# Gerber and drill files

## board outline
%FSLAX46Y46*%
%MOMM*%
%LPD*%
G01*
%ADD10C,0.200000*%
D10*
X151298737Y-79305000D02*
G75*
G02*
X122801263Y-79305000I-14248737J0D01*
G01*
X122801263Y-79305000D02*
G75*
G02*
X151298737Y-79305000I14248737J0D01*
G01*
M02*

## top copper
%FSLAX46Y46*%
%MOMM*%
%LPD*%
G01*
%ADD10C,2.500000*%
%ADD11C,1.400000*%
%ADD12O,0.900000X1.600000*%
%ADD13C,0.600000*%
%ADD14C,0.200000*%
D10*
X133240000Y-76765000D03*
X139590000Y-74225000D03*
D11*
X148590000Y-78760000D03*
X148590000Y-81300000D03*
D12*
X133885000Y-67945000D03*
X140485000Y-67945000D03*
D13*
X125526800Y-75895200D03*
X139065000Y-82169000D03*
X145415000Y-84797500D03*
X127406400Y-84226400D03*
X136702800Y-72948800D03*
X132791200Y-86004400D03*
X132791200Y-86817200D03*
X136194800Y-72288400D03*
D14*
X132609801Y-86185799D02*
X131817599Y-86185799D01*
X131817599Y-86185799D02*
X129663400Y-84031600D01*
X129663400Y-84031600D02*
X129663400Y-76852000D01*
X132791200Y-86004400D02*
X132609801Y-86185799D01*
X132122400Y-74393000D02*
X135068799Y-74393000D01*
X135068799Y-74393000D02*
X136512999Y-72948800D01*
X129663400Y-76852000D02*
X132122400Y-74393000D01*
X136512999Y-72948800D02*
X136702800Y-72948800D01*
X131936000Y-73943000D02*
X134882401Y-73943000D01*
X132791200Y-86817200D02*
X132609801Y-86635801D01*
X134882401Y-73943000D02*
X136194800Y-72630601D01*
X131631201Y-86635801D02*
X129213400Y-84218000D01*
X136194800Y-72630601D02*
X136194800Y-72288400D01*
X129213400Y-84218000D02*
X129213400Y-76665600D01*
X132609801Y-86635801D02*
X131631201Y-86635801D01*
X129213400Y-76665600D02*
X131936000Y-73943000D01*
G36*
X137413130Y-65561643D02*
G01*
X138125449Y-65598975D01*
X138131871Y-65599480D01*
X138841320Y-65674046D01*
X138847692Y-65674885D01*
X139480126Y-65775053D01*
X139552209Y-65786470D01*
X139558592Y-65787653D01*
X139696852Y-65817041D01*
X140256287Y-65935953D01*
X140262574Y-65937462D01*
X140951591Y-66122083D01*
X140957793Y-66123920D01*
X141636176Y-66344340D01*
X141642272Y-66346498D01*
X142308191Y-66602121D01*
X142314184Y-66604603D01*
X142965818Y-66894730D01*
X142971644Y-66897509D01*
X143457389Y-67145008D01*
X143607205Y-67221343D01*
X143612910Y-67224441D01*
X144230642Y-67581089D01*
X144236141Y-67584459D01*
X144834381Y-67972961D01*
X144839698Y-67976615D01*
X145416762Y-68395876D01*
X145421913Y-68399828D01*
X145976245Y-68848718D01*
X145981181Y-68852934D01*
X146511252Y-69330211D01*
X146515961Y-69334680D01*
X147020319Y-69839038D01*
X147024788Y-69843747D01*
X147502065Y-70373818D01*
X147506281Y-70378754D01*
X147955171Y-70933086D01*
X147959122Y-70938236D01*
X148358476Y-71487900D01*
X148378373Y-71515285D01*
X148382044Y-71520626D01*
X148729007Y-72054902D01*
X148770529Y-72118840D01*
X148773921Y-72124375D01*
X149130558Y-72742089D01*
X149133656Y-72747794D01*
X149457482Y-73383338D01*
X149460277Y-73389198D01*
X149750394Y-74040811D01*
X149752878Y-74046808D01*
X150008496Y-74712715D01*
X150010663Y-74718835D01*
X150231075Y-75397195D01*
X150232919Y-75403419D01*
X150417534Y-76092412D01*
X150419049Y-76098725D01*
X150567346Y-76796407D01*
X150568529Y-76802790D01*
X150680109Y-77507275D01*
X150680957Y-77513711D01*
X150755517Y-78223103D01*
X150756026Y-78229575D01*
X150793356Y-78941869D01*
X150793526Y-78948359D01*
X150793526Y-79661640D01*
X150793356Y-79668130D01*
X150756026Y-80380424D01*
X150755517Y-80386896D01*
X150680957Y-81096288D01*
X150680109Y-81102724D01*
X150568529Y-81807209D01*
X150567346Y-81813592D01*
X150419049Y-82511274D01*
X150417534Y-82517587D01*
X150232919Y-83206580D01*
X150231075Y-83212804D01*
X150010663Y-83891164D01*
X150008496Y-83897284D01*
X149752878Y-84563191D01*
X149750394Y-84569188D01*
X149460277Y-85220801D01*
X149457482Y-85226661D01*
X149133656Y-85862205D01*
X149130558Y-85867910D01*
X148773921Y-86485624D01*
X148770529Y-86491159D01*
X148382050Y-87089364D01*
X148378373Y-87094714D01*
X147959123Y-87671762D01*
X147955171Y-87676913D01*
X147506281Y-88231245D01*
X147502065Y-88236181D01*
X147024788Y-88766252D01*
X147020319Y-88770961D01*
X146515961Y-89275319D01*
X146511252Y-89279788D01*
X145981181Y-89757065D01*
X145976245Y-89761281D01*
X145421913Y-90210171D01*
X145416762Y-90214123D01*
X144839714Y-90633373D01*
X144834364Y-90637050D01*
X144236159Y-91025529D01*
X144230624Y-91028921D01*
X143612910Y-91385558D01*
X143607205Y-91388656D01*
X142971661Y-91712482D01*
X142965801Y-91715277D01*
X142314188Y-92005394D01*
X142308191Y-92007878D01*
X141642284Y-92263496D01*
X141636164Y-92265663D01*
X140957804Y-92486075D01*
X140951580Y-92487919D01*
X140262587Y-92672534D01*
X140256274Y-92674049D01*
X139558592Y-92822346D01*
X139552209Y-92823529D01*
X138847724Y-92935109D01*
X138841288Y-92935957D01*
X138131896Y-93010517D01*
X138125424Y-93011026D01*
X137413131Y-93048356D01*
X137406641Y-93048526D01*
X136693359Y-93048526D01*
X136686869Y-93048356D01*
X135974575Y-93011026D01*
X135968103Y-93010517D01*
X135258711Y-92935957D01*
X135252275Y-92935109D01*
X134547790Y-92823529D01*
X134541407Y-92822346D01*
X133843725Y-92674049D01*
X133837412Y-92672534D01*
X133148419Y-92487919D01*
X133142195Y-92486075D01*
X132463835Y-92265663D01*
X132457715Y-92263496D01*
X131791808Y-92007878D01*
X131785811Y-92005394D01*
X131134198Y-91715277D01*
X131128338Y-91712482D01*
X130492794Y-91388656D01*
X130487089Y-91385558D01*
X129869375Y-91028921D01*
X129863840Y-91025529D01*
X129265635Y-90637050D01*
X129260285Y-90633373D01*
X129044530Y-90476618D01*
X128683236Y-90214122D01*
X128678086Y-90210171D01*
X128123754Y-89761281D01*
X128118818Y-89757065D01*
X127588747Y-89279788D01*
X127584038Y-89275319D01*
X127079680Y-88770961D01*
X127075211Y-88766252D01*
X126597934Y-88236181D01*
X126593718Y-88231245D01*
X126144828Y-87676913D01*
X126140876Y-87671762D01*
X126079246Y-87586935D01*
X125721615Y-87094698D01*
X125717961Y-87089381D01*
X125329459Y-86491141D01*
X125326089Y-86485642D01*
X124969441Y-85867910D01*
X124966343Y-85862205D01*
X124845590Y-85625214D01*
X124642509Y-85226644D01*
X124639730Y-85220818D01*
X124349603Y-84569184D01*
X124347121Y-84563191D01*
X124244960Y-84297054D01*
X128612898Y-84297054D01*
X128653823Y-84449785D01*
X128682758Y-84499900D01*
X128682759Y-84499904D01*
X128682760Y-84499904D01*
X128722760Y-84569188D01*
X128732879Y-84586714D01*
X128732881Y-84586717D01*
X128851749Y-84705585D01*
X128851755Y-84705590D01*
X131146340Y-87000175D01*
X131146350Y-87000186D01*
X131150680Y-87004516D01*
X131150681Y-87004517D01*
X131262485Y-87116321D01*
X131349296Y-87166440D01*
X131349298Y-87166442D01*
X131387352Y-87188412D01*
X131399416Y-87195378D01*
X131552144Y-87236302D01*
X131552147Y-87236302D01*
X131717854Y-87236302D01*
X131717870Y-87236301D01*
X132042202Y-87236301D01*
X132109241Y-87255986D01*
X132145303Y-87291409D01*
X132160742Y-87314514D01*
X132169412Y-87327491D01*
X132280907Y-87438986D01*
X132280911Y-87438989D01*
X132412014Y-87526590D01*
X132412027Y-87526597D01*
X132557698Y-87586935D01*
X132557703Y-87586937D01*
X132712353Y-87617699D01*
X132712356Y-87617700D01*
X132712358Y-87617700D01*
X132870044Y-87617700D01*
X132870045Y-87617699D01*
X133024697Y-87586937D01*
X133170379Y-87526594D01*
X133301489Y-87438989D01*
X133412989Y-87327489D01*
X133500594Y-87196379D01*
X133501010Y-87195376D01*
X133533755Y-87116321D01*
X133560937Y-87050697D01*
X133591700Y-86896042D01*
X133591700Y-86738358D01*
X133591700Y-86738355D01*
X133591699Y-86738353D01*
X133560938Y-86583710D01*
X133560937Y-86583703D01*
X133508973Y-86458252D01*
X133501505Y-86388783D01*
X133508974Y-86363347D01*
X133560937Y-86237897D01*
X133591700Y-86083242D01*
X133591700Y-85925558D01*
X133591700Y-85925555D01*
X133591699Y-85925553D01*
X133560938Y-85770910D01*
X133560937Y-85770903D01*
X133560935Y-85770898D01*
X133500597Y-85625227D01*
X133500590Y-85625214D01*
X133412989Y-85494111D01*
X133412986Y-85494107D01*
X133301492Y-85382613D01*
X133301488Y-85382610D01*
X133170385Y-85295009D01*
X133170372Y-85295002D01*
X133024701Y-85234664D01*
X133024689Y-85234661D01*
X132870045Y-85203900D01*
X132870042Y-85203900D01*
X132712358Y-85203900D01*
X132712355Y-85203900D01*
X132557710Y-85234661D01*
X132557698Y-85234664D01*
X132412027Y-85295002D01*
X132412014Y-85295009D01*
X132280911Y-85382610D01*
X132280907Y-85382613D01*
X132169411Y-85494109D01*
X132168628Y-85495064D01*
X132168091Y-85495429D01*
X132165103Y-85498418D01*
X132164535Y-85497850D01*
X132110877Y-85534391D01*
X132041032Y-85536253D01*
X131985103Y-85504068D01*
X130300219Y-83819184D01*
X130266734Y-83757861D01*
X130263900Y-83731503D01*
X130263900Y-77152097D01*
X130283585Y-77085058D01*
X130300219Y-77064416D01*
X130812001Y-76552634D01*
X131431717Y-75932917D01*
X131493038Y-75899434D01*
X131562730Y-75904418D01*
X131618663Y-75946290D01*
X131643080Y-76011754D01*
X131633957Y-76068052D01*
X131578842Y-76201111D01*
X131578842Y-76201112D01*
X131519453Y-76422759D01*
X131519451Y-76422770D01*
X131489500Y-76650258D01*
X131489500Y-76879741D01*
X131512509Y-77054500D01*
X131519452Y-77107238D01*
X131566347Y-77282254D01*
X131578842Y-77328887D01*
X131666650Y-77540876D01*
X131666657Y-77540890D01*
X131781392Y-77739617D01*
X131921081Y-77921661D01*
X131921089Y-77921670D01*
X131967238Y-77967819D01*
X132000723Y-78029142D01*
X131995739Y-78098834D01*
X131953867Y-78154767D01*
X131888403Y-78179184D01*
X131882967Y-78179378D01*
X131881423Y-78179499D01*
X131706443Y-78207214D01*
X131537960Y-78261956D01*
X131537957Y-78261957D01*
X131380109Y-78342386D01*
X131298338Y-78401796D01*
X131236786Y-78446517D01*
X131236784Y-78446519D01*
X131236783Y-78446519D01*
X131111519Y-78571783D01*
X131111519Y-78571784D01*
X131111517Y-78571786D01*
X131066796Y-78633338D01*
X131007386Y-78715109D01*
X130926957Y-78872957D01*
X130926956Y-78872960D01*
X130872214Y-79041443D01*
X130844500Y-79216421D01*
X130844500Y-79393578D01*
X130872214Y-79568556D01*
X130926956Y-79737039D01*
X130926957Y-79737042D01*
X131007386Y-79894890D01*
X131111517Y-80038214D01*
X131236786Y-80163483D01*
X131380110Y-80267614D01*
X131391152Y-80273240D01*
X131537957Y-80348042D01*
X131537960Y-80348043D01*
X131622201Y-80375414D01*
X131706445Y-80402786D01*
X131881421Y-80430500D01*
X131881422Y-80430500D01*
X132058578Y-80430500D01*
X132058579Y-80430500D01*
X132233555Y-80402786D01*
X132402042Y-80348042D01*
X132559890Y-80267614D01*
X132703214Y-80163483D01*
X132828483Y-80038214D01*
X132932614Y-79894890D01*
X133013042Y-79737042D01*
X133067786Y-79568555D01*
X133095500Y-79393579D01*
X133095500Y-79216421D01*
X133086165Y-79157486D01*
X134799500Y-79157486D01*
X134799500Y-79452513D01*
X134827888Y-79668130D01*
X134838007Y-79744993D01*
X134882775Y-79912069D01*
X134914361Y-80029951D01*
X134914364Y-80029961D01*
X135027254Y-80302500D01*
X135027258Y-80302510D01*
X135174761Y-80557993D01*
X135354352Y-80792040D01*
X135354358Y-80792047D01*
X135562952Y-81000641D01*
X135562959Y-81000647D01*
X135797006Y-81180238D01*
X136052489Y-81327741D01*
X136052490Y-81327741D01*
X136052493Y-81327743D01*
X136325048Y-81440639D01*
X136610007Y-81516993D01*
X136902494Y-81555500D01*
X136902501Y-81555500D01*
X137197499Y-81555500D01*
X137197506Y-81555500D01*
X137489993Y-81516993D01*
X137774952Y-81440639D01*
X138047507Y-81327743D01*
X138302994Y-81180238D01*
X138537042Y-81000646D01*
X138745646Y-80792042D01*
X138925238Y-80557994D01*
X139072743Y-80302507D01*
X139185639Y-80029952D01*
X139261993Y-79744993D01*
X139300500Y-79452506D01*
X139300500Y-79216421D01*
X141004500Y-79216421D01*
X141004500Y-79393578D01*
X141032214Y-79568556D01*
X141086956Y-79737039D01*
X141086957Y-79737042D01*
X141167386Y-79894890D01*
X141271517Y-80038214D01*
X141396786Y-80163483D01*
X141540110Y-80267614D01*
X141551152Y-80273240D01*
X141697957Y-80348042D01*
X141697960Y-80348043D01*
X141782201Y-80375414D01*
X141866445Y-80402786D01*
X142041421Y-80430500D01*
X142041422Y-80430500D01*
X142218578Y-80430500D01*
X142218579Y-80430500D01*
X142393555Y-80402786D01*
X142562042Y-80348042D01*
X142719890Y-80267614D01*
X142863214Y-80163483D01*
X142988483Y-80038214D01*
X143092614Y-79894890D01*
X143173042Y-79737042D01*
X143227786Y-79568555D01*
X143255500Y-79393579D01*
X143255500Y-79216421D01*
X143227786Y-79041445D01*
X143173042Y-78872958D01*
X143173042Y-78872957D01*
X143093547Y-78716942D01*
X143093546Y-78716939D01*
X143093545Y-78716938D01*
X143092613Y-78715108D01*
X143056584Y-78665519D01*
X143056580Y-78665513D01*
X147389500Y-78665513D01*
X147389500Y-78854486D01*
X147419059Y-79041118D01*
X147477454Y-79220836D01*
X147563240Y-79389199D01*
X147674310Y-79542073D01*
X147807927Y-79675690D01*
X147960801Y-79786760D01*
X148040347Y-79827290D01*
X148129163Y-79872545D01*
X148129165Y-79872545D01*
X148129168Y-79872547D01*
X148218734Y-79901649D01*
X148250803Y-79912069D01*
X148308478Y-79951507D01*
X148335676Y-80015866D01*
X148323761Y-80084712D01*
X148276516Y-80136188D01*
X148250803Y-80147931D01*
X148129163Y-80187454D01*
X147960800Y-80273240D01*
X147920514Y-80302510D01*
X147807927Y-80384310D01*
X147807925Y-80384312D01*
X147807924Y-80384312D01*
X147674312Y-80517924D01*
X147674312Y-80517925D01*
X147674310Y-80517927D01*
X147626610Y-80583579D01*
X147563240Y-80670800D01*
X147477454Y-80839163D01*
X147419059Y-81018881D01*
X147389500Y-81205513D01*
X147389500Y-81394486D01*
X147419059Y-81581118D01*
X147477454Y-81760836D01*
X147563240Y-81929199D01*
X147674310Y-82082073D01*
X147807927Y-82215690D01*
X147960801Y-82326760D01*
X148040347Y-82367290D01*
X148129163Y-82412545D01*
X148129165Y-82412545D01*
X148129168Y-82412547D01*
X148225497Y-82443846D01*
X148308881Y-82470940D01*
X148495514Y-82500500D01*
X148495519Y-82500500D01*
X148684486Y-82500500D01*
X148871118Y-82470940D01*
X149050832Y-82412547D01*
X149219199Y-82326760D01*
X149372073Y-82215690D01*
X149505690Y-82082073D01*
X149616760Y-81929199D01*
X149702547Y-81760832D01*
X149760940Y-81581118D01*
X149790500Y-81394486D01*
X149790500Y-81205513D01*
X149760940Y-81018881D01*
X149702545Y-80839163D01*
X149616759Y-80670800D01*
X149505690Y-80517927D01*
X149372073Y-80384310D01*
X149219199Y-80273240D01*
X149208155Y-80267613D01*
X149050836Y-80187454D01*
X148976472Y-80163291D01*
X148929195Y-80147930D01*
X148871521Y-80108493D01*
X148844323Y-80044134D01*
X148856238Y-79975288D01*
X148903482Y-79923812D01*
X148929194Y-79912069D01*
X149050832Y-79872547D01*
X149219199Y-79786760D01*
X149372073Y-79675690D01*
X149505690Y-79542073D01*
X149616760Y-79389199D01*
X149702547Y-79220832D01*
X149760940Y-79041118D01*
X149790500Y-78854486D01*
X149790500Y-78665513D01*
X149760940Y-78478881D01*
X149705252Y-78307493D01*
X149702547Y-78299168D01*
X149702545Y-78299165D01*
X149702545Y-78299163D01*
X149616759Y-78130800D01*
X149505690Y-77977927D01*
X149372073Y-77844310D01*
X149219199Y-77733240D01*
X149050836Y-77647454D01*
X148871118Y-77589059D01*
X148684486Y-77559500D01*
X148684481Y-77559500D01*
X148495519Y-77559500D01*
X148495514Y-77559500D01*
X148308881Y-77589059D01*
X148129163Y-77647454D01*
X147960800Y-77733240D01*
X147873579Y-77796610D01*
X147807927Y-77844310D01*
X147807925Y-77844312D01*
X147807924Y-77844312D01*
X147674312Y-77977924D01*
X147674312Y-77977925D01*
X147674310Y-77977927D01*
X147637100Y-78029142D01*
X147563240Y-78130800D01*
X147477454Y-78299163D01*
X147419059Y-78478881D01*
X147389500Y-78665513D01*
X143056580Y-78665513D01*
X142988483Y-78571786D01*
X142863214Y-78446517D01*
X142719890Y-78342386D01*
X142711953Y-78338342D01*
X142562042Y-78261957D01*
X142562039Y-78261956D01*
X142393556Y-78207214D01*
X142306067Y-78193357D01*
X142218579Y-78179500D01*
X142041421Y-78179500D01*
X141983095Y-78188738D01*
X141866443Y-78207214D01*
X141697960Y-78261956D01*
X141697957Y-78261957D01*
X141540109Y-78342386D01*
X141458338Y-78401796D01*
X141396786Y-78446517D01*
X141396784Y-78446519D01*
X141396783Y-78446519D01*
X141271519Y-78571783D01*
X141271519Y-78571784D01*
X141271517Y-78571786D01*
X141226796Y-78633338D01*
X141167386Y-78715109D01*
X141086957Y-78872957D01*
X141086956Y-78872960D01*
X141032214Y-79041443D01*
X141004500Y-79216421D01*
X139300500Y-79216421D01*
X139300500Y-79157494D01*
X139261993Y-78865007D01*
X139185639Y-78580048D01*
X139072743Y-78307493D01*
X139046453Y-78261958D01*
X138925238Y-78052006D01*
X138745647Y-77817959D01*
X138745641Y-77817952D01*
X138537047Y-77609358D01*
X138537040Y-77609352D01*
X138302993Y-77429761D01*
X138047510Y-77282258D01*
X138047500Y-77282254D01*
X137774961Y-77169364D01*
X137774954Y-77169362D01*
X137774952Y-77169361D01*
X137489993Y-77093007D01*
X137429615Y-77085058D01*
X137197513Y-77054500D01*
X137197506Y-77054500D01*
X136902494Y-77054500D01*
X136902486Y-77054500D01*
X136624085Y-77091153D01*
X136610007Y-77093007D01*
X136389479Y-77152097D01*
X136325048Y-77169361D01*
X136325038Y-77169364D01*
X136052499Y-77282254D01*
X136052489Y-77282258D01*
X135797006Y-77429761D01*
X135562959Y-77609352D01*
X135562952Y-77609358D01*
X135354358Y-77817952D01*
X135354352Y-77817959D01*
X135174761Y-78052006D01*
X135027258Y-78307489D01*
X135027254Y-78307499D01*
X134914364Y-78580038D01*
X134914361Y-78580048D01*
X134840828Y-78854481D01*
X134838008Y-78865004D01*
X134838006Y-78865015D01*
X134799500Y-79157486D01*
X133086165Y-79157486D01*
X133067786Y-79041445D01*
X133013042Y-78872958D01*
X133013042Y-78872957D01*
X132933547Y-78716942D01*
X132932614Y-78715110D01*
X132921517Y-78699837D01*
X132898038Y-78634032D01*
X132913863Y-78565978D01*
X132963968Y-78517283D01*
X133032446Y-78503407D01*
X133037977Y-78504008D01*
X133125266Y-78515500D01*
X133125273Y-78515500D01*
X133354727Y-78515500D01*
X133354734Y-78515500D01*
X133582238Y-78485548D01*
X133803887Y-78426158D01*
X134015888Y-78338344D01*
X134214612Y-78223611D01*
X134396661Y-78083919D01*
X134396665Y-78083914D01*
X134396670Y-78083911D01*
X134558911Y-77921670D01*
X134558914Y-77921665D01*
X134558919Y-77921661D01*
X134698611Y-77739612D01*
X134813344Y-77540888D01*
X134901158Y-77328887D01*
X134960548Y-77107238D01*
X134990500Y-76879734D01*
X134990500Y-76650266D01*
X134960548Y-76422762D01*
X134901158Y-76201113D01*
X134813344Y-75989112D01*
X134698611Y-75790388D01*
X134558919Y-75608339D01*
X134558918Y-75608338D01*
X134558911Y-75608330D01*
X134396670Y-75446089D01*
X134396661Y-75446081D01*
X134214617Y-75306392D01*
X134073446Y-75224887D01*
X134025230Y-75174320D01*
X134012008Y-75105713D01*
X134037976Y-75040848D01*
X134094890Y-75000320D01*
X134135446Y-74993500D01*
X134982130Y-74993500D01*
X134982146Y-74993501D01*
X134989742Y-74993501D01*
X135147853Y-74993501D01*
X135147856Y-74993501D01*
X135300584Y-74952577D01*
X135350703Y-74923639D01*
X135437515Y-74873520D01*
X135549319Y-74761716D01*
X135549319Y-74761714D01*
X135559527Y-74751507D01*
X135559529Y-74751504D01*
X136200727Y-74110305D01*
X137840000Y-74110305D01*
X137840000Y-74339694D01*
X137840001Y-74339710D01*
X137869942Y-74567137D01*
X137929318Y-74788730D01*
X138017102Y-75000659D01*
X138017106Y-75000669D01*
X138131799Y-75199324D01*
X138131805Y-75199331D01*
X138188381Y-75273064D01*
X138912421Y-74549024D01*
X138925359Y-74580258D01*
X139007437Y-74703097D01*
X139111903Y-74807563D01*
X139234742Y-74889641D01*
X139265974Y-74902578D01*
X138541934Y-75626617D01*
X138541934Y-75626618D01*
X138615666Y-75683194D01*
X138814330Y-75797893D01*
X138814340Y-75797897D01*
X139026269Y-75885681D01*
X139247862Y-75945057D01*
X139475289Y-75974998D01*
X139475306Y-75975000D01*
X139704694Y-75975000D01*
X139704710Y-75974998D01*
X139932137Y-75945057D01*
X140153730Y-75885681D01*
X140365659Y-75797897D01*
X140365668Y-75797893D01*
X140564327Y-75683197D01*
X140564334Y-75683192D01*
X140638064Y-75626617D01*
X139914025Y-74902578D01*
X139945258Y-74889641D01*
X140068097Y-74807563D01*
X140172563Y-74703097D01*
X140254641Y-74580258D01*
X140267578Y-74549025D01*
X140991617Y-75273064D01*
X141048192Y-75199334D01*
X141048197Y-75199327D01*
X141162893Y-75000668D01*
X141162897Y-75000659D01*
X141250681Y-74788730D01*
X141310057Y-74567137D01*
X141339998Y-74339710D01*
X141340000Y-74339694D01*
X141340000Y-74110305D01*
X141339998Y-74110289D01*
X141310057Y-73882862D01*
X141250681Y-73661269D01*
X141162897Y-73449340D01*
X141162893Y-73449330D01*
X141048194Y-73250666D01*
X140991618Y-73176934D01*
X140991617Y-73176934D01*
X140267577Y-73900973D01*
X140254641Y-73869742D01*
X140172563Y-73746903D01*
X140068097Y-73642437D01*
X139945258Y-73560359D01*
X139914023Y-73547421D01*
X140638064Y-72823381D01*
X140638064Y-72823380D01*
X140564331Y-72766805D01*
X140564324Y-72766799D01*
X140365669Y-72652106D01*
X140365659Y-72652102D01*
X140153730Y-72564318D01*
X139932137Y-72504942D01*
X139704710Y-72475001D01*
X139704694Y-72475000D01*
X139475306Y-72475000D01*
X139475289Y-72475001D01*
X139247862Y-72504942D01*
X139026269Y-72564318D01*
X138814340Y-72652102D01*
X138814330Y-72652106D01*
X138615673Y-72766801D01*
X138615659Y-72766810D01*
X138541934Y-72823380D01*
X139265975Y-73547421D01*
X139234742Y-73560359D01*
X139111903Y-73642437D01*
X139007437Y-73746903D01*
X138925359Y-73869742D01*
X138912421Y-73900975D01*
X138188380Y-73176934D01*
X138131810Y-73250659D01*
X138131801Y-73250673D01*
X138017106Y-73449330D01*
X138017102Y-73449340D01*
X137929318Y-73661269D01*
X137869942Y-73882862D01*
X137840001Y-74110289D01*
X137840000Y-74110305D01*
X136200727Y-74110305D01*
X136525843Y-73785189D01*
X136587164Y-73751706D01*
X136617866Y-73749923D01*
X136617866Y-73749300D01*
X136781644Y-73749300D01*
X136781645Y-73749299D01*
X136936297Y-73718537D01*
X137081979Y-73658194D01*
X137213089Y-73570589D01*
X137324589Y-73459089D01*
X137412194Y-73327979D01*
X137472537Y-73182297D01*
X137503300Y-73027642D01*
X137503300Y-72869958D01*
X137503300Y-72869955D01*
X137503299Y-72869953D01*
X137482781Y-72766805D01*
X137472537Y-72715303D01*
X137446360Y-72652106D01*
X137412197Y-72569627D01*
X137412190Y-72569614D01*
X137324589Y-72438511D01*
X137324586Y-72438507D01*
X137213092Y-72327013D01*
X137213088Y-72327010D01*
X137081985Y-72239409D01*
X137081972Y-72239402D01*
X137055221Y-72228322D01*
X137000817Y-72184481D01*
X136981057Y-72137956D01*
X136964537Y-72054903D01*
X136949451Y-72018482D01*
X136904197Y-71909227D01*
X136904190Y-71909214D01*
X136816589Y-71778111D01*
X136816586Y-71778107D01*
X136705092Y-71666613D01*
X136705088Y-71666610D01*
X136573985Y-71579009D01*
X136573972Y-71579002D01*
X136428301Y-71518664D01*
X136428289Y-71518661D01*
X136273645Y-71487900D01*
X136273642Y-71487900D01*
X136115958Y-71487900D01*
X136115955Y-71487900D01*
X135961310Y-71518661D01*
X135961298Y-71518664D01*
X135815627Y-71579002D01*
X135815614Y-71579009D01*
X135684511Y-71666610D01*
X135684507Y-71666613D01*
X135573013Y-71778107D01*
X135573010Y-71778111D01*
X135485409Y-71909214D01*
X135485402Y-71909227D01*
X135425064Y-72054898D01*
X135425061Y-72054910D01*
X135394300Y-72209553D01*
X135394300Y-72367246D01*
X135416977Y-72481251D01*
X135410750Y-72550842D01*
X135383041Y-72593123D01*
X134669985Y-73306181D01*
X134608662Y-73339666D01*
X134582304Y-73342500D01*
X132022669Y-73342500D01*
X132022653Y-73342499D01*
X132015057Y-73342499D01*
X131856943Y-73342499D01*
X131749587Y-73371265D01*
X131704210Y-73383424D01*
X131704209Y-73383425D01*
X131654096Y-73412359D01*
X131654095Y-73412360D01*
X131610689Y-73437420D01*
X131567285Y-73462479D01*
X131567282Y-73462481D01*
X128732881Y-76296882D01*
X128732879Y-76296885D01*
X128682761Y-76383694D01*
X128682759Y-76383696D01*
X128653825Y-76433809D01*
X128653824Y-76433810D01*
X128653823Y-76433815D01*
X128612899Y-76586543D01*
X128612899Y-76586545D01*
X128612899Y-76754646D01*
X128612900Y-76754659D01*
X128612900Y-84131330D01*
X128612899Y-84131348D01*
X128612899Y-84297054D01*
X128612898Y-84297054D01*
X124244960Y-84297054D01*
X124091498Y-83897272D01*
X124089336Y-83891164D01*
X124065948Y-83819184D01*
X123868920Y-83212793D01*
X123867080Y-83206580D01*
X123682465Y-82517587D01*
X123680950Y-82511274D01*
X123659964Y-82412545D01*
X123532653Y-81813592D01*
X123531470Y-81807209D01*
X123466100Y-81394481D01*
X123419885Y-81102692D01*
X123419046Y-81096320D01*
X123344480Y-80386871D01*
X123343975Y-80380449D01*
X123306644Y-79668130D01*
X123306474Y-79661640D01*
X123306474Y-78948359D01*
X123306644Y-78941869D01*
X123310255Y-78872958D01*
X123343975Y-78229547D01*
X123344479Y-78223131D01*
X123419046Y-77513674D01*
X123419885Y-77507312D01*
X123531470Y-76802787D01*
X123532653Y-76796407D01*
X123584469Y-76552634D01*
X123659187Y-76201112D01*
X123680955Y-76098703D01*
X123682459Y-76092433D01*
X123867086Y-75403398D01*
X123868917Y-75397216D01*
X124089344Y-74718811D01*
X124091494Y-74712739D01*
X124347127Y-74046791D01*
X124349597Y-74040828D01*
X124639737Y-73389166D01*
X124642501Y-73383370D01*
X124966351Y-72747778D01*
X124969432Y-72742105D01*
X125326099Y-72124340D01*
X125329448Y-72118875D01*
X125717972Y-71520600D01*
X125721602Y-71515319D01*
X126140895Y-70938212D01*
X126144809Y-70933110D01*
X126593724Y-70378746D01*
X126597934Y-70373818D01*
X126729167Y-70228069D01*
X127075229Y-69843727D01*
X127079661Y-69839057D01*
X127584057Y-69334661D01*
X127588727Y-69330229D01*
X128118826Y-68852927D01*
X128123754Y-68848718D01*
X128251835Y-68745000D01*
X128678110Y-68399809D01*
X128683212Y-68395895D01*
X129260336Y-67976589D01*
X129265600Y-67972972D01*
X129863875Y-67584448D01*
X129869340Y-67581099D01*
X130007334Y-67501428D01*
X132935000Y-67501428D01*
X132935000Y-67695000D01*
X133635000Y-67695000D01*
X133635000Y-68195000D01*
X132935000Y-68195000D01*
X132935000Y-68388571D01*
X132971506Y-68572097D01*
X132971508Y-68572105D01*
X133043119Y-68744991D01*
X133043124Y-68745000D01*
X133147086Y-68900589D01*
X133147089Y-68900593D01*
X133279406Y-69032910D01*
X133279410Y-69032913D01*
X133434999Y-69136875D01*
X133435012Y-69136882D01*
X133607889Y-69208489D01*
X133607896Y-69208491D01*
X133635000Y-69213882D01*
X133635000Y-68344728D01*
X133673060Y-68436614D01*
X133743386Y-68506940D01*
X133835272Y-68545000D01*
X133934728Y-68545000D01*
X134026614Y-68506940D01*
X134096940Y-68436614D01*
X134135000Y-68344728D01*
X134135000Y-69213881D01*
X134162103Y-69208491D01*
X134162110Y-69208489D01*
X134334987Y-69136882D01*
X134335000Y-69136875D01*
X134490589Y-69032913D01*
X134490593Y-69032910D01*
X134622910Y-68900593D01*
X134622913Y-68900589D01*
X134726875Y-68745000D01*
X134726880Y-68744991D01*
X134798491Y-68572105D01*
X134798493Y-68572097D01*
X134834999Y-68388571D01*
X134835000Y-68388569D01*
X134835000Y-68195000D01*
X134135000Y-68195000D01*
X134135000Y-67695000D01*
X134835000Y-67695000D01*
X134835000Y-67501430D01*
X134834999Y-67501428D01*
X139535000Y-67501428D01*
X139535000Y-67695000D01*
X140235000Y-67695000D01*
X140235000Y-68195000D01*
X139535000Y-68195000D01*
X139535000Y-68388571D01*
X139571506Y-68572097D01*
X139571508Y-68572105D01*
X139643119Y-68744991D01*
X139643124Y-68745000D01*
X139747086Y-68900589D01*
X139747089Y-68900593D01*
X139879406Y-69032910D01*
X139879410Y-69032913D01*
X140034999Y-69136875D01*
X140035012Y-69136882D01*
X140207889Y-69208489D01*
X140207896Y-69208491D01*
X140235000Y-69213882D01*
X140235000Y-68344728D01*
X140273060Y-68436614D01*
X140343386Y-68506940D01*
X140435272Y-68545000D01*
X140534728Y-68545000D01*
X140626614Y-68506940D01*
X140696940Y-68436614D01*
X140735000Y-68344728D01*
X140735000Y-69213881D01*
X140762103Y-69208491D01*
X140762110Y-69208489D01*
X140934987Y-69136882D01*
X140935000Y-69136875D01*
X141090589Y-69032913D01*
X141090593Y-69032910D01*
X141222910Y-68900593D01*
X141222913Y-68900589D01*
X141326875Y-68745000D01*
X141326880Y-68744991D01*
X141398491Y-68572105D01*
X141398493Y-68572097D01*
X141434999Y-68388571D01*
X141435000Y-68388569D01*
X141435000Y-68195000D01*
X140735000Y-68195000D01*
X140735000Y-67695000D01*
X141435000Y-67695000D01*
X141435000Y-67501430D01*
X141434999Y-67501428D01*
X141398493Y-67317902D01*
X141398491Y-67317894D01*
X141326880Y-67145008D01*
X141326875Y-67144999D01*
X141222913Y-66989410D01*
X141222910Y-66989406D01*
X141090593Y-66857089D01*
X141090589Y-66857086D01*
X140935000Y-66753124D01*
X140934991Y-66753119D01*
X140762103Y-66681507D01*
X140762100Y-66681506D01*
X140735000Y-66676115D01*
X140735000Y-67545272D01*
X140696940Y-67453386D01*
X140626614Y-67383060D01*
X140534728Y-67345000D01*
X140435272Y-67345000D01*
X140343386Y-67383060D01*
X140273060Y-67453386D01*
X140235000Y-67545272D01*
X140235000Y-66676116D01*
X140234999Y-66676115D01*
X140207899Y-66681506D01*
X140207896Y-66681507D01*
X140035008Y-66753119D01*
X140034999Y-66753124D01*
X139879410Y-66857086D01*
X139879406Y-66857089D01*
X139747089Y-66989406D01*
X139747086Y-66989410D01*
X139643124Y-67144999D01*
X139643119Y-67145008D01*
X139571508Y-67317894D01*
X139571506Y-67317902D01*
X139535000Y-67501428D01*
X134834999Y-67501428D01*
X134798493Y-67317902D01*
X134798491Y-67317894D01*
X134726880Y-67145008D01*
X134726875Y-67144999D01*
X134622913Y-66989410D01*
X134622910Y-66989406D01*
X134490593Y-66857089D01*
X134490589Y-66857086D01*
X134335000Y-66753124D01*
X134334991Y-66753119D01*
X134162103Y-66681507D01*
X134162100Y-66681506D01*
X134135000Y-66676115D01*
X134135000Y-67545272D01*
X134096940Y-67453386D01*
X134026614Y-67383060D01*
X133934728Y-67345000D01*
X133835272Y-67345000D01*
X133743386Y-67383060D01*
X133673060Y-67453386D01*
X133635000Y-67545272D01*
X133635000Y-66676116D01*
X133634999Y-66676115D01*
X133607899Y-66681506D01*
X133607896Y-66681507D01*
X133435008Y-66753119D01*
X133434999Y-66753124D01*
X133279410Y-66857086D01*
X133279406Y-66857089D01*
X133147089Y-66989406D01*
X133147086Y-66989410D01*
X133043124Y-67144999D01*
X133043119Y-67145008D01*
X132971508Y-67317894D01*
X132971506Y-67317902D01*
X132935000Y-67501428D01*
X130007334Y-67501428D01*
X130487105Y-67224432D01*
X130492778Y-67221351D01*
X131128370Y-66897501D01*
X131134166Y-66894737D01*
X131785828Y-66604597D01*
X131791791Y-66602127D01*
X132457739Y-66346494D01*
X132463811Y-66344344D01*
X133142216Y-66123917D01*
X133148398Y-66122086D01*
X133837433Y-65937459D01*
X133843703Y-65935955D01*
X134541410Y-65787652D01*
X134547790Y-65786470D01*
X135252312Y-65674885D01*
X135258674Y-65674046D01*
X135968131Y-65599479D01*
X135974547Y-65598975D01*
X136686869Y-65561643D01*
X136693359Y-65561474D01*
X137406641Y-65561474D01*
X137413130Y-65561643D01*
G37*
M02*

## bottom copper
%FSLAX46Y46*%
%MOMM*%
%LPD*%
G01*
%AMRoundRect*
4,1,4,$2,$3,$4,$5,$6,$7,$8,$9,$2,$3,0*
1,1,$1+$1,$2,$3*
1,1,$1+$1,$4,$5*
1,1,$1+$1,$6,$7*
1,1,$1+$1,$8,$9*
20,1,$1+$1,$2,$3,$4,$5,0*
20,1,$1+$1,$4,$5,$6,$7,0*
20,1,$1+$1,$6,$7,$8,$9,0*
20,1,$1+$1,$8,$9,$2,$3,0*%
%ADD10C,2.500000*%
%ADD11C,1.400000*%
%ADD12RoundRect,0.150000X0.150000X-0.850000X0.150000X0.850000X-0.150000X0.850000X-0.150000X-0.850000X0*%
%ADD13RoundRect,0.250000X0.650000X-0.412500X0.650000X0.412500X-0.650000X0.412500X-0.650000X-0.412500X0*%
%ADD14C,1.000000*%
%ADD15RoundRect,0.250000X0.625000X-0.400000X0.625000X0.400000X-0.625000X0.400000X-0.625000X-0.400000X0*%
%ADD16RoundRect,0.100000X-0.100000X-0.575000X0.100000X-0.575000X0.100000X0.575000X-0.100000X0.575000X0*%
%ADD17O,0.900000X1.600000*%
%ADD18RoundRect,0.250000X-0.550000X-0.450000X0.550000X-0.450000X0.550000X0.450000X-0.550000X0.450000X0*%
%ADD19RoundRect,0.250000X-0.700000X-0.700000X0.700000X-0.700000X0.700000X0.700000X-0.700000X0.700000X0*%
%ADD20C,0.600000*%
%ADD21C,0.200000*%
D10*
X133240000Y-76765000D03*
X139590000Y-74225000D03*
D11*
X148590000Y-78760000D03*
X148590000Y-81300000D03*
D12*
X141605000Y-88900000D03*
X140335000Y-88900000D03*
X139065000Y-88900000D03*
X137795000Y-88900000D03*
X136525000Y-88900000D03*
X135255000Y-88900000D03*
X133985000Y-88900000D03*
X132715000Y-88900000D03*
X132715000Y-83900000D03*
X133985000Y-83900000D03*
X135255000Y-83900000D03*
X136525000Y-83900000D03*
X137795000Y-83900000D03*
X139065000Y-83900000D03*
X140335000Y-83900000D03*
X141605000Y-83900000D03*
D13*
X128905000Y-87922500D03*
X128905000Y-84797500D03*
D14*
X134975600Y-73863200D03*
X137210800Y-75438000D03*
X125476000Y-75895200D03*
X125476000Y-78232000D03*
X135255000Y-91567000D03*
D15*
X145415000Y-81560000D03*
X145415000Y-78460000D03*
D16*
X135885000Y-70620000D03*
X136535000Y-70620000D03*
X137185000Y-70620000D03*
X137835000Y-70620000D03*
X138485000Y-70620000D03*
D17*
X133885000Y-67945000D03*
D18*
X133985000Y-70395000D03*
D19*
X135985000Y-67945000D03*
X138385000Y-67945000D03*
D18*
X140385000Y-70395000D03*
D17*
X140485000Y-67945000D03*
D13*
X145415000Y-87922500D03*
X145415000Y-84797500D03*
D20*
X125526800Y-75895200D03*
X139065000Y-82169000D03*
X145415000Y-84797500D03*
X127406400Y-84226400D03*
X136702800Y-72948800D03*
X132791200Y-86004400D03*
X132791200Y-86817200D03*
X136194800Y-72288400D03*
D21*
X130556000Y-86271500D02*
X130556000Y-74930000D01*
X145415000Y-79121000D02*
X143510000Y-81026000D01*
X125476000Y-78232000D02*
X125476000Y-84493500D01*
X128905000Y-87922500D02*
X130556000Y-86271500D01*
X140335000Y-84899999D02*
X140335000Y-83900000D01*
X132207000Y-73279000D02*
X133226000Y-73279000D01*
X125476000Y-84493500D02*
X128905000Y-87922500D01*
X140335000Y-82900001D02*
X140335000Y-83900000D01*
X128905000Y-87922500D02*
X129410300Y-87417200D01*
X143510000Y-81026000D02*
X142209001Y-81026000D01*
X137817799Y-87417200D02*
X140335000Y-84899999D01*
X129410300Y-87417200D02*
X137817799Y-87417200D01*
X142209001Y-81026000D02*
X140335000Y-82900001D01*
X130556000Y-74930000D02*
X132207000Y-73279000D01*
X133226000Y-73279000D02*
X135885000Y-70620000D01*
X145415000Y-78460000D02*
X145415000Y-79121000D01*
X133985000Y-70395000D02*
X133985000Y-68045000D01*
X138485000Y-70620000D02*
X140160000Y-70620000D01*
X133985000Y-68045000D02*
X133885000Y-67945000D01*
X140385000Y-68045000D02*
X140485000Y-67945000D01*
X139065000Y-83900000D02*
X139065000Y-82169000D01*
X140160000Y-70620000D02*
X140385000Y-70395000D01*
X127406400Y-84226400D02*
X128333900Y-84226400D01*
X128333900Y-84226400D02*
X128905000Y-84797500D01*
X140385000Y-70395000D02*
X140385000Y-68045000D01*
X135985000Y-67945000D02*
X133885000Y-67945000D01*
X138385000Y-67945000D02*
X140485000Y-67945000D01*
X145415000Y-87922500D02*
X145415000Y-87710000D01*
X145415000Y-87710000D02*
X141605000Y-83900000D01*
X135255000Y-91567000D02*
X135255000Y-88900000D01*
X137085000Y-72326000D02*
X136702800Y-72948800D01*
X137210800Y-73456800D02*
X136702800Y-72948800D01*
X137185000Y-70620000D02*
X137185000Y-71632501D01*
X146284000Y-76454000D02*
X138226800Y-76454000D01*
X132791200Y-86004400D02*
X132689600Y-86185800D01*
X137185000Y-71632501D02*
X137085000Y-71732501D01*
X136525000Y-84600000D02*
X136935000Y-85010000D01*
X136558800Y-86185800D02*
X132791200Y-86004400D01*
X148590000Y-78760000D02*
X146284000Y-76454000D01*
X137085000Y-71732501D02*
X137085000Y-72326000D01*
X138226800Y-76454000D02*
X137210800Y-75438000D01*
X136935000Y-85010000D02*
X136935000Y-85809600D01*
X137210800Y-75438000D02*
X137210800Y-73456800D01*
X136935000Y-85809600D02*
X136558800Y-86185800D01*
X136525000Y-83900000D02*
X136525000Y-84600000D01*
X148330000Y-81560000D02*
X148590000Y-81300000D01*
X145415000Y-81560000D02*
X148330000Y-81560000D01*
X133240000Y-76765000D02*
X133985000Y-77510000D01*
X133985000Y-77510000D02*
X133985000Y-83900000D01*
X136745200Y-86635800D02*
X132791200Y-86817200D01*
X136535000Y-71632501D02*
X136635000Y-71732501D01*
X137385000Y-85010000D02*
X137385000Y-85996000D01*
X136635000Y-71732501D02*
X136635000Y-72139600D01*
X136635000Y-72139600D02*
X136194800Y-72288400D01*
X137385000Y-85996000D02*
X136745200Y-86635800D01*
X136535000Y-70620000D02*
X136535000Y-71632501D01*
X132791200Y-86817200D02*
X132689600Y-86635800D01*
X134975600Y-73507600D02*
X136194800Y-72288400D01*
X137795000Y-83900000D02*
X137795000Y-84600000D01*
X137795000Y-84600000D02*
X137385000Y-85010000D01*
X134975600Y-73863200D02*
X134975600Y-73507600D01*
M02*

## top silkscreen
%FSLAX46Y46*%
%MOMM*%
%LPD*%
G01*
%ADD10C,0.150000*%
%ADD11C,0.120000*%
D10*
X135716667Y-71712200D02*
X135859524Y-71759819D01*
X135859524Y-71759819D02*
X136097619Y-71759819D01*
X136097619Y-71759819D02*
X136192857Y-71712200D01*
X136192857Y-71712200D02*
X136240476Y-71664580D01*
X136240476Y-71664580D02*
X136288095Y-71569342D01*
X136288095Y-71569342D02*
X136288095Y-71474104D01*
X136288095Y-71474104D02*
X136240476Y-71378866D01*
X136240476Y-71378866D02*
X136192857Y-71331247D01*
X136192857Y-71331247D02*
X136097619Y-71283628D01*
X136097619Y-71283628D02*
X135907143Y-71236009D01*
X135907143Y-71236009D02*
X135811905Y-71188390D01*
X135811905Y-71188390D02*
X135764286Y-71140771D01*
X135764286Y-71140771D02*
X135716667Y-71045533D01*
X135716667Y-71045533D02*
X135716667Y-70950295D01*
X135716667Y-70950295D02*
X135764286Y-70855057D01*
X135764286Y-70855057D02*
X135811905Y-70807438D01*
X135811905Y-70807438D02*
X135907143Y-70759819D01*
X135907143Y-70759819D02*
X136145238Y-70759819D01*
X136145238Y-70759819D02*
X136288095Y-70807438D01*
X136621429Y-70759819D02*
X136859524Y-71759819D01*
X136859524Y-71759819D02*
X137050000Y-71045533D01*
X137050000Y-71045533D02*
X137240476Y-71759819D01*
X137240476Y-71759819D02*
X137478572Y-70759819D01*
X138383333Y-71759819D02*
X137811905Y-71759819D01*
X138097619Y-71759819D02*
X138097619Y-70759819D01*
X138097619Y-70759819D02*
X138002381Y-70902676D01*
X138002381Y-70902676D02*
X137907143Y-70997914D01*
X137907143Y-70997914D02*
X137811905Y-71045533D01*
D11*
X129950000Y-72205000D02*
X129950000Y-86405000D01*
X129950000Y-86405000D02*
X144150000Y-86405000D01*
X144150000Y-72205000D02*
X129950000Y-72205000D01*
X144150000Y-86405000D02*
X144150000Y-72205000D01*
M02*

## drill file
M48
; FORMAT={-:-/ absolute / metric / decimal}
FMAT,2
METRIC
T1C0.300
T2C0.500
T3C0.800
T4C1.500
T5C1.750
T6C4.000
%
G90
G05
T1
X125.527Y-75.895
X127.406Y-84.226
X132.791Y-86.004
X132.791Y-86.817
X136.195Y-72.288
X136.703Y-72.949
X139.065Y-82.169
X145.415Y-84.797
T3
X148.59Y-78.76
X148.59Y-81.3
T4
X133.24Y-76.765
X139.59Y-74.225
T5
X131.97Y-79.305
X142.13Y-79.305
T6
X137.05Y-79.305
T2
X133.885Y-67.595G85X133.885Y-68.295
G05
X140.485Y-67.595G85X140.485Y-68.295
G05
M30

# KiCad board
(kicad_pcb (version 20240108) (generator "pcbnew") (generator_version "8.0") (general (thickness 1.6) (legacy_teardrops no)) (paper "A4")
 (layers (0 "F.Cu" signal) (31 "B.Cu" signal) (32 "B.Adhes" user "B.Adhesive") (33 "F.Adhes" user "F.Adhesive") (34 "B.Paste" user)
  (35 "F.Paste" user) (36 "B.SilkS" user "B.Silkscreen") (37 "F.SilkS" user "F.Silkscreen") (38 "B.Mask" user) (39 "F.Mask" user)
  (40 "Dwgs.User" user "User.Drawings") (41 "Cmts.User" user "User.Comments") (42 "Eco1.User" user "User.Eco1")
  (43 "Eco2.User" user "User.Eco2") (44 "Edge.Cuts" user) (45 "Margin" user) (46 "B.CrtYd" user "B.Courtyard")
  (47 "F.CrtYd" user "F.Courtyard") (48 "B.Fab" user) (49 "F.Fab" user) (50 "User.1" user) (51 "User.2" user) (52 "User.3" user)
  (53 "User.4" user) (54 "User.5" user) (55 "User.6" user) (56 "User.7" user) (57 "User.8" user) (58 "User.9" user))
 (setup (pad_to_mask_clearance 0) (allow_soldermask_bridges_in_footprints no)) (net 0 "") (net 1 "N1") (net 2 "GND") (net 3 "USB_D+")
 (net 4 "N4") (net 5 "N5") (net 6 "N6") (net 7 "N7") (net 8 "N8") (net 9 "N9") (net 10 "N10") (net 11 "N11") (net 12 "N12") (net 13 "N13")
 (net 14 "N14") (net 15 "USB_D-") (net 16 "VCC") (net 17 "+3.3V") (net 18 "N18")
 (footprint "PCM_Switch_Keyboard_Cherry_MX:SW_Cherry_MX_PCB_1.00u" (layer "F.Cu") (at 137.05 79.305)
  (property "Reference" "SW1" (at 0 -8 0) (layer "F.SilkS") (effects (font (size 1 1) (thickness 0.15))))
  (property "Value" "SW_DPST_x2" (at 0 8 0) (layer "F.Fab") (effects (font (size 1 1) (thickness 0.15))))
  (fp_line (start -7.1 -7.1) (end -7.1 7.1) (stroke (width 0.12) (type solid)) (layer "F.SilkS"))
  (fp_line (start -7.1 7.1) (end 7.1 7.1) (stroke (width 0.12) (type solid)) (layer "F.SilkS"))
  (fp_line (start 7.1 -7.1) (end -7.1 -7.1) (stroke (width 0.12) (type solid)) (layer "F.SilkS"))
  (fp_line (start 7.1 7.1) (end 7.1 -7.1) (stroke (width 0.12) (type solid)) (layer "F.SilkS"))
  (pad "" np_thru_hole circle (at -5.08 0) (size 1.75 1.75) (drill 1.75) (layers "*.Cu" "*.Mask"))
  (pad "" np_thru_hole circle (at 0 0) (size 4 4) (drill 4) (layers "*.Cu" "*.Mask"))
  (pad "" np_thru_hole circle (at 5.08 0) (size 1.75 1.75) (drill 1.75) (layers "*.Cu" "*.Mask"))
  (pad "1" thru_hole circle (at -3.81 -2.54) (size 2.5 2.5) (drill 1.5) (layers "*.Cu" "*.Mask") (remove_unused_layers no) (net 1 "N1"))
  (pad "2" thru_hole circle (at 2.54 -5.08) (size 2.5 2.5) (drill 1.5) (layers "*.Cu" "*.Mask") (remove_unused_layers no) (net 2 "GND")))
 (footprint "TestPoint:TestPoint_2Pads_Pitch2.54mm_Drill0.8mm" (layer "B.Cu") (at 148.59 78.76 -90)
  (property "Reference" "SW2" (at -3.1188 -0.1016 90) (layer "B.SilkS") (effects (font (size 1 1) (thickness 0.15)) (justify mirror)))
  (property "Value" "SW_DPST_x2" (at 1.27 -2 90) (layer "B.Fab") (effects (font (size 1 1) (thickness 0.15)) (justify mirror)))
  (pad "1" thru_hole circle (at 0 0 270) (size 1.4 1.4) (drill 0.8) (layers "*.Cu" "*.Mask") (remove_unused_layers no) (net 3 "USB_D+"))
  (pad "2" thru_hole circle (at 2.54 0 270) (size 1.4 1.4) (drill 0.8) (layers "*.Cu" "*.Mask") (remove_unused_layers no) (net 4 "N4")))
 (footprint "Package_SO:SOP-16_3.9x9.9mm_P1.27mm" (layer "B.Cu") (at 137.16 86.4 90)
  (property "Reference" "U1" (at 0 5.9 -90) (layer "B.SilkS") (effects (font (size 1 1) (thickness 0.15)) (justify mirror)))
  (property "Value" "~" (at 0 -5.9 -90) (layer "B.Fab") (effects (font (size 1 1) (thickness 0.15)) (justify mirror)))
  (pad "1" smd roundrect (at -2.5 4.445 90) (size 2 0.6) (layers "B.Cu" "B.Paste" "B.Mask") (roundrect_rratio 0.25) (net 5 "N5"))
  (pad "2" smd roundrect (at -2.5 3.175 90) (size 2 0.6) (layers "B.Cu" "B.Paste" "B.Mask") (roundrect_rratio 0.25) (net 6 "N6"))
  (pad "3" smd roundrect (at -2.5 1.905 90) (size 2 0.6) (layers "B.Cu" "B.Paste" "B.Mask") (roundrect_rratio 0.25) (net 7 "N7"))
  (pad "4" smd roundrect (at -2.5 0.635 90) (size 2 0.6) (layers "B.Cu" "B.Paste" "B.Mask") (roundrect_rratio 0.25) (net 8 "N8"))
  (pad "5" smd roundrect (at -2.5 -0.635 90) (size 2 0.6) (layers "B.Cu" "B.Paste" "B.Mask") (roundrect_rratio 0.25) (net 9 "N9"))
  (pad "6" smd roundrect (at -2.5 -1.905 90) (size 2 0.6) (layers "B.Cu" "B.Paste" "B.Mask") (roundrect_rratio 0.25) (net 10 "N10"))
  (pad "7" smd roundrect (at -2.5 -3.175 90) (size 2 0.6) (layers "B.Cu" "B.Paste" "B.Mask") (roundrect_rratio 0.25) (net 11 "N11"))
  (pad "8" smd roundrect (at -2.5 -4.445 90) (size 2 0.6) (layers "B.Cu" "B.Paste" "B.Mask") (roundrect_rratio 0.25) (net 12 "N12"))
  (pad "9" smd roundrect (at 2.5 -4.445 90) (size 2 0.6) (layers "B.Cu" "B.Paste" "B.Mask") (roundrect_rratio 0.25) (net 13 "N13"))
  (pad "10" smd roundrect (at 2.5 -3.175 90) (size 2 0.6) (layers "B.Cu" "B.Paste" "B.Mask") (roundrect_rratio 0.25) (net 1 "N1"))
  (pad "11" smd roundrect (at 2.5 -1.905 90) (size 2 0.6) (layers "B.Cu" "B.Paste" "B.Mask") (roundrect_rratio 0.25) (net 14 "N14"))
  (pad "12" smd roundrect (at 2.5 -0.635 90) (size 2 0.6) (layers "B.Cu" "B.Paste" "B.Mask") (roundrect_rratio 0.25) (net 3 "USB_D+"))
  (pad "13" smd roundrect (at 2.5 0.635 90) (size 2 0.6) (layers "B.Cu" "B.Paste" "B.Mask") (roundrect_rratio 0.25) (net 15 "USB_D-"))
  (pad "14" smd roundrect (at 2.5 1.905 90) (size 2 0.6) (layers "B.Cu" "B.Paste" "B.Mask") (roundrect_rratio 0.25) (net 2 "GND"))
  (pad "15" smd roundrect (at 2.5 3.175 90) (size 2 0.6) (layers "B.Cu" "B.Paste" "B.Mask") (roundrect_rratio 0.25) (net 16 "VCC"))
  (pad "16" smd roundrect (at 2.5 4.445 90) (size 2 0.6) (layers "B.Cu" "B.Paste" "B.Mask") (roundrect_rratio 0.25) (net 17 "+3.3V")))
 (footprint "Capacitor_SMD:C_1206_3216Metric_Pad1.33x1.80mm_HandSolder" (layer "B.Cu") (at 128.905 86.36 90)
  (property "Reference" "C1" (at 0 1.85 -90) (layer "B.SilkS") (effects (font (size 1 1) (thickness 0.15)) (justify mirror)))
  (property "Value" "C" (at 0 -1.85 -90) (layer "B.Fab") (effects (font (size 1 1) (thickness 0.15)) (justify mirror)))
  (pad "1" smd roundrect (at -1.5625 0 90) (size 1.325 1.8) (layers "B.Cu" "B.Paste" "B.Mask") (roundrect_rratio 0.188679) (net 16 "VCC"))
  (pad "2" smd roundrect (at 1.5625 0 90) (size 1.325 1.8) (layers "B.Cu" "B.Paste" "B.Mask") (roundrect_rratio 0.188679) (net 2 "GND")))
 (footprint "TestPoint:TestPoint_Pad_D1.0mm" (layer "B.Cu") (at 134.9756 73.8632 180)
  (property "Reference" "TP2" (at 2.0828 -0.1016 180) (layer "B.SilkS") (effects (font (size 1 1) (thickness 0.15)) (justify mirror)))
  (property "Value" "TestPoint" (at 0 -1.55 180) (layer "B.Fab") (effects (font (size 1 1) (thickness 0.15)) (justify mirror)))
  (pad "1" smd circle (at 0 0 180) (size 1 1) (layers "B.Cu" "B.Mask") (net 15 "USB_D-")))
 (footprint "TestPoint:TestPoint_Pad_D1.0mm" (layer "B.Cu") (at 137.2108 75.438 180)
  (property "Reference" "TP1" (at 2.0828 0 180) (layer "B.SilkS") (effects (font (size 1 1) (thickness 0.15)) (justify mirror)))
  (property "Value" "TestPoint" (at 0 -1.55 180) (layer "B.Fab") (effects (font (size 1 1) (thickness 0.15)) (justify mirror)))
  (pad "1" smd circle (at 0 0 180) (size 1 1) (layers "B.Cu" "B.Mask") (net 3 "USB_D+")))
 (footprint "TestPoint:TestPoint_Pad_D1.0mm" (layer "B.Cu") (at 125.476 75.8952 180)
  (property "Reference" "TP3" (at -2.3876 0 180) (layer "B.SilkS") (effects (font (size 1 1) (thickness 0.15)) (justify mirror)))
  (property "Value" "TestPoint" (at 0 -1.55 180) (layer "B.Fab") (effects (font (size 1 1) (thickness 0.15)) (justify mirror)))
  (pad "1" smd circle (at 0 0 180) (size 1 1) (layers "B.Cu" "B.Mask") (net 2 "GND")))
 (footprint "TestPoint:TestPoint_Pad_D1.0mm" (layer "B.Cu") (at 125.476 78.232 180)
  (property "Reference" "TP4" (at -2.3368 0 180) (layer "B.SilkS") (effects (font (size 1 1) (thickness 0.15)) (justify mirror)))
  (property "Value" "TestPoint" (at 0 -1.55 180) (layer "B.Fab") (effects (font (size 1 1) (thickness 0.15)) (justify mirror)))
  (pad "1" smd circle (at 0 0 180) (size 1 1) (layers "B.Cu" "B.Mask") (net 16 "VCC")))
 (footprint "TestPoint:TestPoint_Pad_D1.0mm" (layer "B.Cu") (at 135.255 91.567 180)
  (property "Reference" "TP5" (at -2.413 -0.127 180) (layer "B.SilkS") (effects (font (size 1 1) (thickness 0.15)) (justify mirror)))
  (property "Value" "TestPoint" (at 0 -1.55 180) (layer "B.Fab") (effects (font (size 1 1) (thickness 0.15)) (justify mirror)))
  (pad "1" smd circle (at 0 0 180) (size 1 1) (layers "B.Cu" "B.Mask") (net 10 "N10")))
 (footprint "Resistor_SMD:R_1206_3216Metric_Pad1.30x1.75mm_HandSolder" (layer "B.Cu") (at 145.415 80.01 90)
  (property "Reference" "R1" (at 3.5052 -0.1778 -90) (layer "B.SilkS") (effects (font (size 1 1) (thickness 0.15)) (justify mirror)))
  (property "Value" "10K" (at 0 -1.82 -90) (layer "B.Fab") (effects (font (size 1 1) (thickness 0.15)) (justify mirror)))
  (pad "1" smd roundrect (at -1.55 0 90) (size 1.3 1.75) (layers "B.Cu" "B.Paste" "B.Mask") (roundrect_rratio 0.192308) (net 4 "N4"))
  (pad "2" smd roundrect (at 1.55 0 90) (size 1.3 1.75) (layers "B.Cu" "B.Paste" "B.Mask") (roundrect_rratio 0.192308) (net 16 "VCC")))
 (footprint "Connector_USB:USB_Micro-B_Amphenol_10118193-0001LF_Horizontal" (layer "B.Cu") (at 137.185 67.945)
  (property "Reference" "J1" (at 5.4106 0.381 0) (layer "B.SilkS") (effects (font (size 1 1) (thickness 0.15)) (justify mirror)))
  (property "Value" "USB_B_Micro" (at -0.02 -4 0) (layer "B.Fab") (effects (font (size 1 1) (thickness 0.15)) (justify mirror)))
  (pad "1" smd roundrect (at -1.3 2.675) (size 0.4 1.35) (layers "B.Cu" "B.Paste" "B.Mask") (roundrect_rratio 0.25) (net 16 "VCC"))
  (pad "2" smd roundrect (at -0.65 2.675) (size 0.4 1.35) (layers "B.Cu" "B.Paste" "B.Mask") (roundrect_rratio 0.25) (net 15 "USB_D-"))
  (pad "3" smd roundrect (at 0 2.675) (size 0.4 1.35) (layers "B.Cu" "B.Paste" "B.Mask") (roundrect_rratio 0.25) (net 3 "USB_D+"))
  (pad "4" smd roundrect (at 0.65 2.675) (size 0.4 1.35) (layers "B.Cu" "B.Paste" "B.Mask") (roundrect_rratio 0.25) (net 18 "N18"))
  (pad "5" smd roundrect (at 1.3 2.675) (size 0.4 1.35) (layers "B.Cu" "B.Paste" "B.Mask") (roundrect_rratio 0.25) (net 2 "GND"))
  (pad "6" thru_hole oval (at -3.3 0 270) (size 1.6 0.9) (drill oval 1.2 0.5) (layers "*.Cu" "*.Mask" "B.Paste") (remove_unused_layers no)
   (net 2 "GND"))
  (pad "6" smd roundrect (at -3.2 2.45) (size 1.6 1.4) (layers "B.Cu" "B.Paste" "B.Mask") (roundrect_rratio 0.1785714286) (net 2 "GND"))
  (pad "6" smd roundrect (at -1.2 0) (size 1.9 1.9) (layers "B.Cu" "B.Paste" "B.Mask") (roundrect_rratio 0.1315789474) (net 2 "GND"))
  (pad "6" smd roundrect (at 1.2 0) (size 1.9 1.9) (layers "B.Cu" "B.Paste" "B.Mask") (roundrect_rratio 0.1315789474) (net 2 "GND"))
  (pad "6" smd roundrect (at 3.2 2.45) (size 1.6 1.4) (layers "B.Cu" "B.Paste" "B.Mask") (roundrect_rratio 0.1785714286) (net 2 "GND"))
  (pad "6" thru_hole oval (at 3.3 0 270) (size 1.6 0.9) (drill oval 1.2 0.5) (layers "*.Cu" "*.Mask" "B.Paste") (remove_unused_layers no)
   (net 2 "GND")))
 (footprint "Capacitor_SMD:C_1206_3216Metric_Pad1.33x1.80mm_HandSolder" (layer "B.Cu") (at 145.415 86.36 90)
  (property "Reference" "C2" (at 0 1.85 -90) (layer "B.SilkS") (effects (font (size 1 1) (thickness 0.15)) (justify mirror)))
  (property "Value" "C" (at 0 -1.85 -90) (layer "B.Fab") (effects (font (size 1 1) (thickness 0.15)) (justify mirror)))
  (pad "1" smd roundrect (at -1.5625 0 90) (size 1.325 1.8) (layers "B.Cu" "B.Paste" "B.Mask") (roundrect_rratio 0.188679) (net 17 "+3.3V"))
  (pad "2" smd roundrect (at 1.5625 0 90) (size 1.325 1.8) (layers "B.Cu" "B.Paste" "B.Mask") (roundrect_rratio 0.188679) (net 2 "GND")))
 (gr_circle (center 137.05 79.305) (end 134.62 93.345) (stroke (width 0.2) (type default)) (fill none) (layer "Edge.Cuts"))
 (segment (start 130.556 86.2715) (end 130.556 74.93) (width 0.2) (layer "B.Cu") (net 16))
 (segment (start 145.415 79.121) (end 143.51 81.026) (width 0.2) (layer "B.Cu") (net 16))
 (segment (start 125.476 78.232) (end 125.476 84.4935) (width 0.2) (layer "B.Cu") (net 16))
 (segment (start 128.905 87.9225) (end 130.556 86.2715) (width 0.2) (layer "B.Cu") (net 16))
 (segment (start 140.335 84.899999) (end 140.335 83.9) (width 0.2) (layer "B.Cu") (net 16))
 (segment (start 132.207 73.279) (end 133.226 73.279) (width 0.2) (layer "B.Cu") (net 16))
 (segment (start 125.476 84.4935) (end 128.905 87.9225) (width 0.2) (layer "B.Cu") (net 16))
 (segment (start 140.335 82.900001) (end 140.335 83.9) (width 0.2) (layer "B.Cu") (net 16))
 (segment (start 128.905 87.9225) (end 129.4103 87.4172) (width 0.2) (layer "B.Cu") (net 16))
 (segment (start 143.51 81.026) (end 142.209001 81.026) (width 0.2) (layer "B.Cu") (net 16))
 (segment (start 137.817799 87.4172) (end 140.335 84.899999) (width 0.2) (layer "B.Cu") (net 16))
 (segment (start 129.4103 87.4172) (end 137.817799 87.4172) (width 0.2) (layer "B.Cu") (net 16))
 (segment (start 142.209001 81.026) (end 140.335 82.900001) (width 0.2) (layer "B.Cu") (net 16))
 (segment (start 130.556 74.93) (end 132.207 73.279) (width 0.2) (layer "B.Cu") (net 16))
 (segment (start 133.226 73.279) (end 135.885 70.62) (width 0.2) (layer "B.Cu") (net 16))
 (segment (start 145.415 78.46) (end 145.415 79.121) (width 0.2) (layer "B.Cu") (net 16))
 (via (at 125.5268 75.8952) (size 0.6) (drill 0.3) (layers "F.Cu" "B.Cu") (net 2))
 (via (at 139.065 82.169) (size 0.6) (drill 0.3) (layers "F.Cu" "B.Cu") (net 2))
 (via (at 145.415 84.7975) (size 0.6) (drill 0.3) (layers "F.Cu" "B.Cu") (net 2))
 (via (at 127.4064 84.2264) (size 0.6) (drill 0.3) (layers "F.Cu" "B.Cu") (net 2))
 (segment (start 133.985 70.395) (end 133.985 68.045) (width 0.2) (layer "B.Cu") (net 2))
 (segment (start 138.485 70.62) (end 140.16 70.62) (width 0.2) (layer "B.Cu") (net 2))
 (segment (start 133.985 68.045) (end 133.885 67.945) (width 0.2) (layer "B.Cu") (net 2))
 (segment (start 140.385 68.045) (end 140.485 67.945) (width 0.2) (layer "B.Cu") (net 2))
 (segment (start 139.065 83.9) (end 139.065 82.169) (width 0.2) (layer "B.Cu") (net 2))
 (segment (start 140.16 70.62) (end 140.385 70.395) (width 0.2) (layer "B.Cu") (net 2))
 (segment (start 127.4064 84.2264) (end 128.3339 84.2264) (width 0.2) (layer "B.Cu") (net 2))
 (segment (start 128.3339 84.2264) (end 128.905 84.7975) (width 0.2) (layer "B.Cu") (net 2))
 (segment (start 140.385 70.395) (end 140.385 68.045) (width 0.2) (layer "B.Cu") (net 2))
 (segment (start 135.985 67.945) (end 133.885 67.945) (width 0.2) (layer "B.Cu") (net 2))
 (segment (start 138.385 67.945) (end 140.485 67.945) (width 0.2) (layer "B.Cu") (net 2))
 (segment (start 145.415 87.9225) (end 145.415 87.71) (width 0.2) (layer "B.Cu") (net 17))
 (segment (start 145.415 87.71) (end 141.605 83.9) (width 0.2) (layer "B.Cu") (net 17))
 (segment (start 135.255 91.567) (end 135.255 88.9) (width 0.2) (layer "B.Cu") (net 10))
 (segment (start 132.609801 86.185799) (end 131.817599 86.185799) (width 0.2) (layer "F.Cu") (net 3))
 (segment (start 131.817599 86.185799) (end 129.6634 84.0316) (width 0.2) (layer "F.Cu") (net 3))
 (segment (start 129.6634 84.0316) (end 129.6634 76.852) (width 0.2) (layer "F.Cu") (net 3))
 (segment (start 132.7912 86.0044) (end 132.609801 86.185799) (width 0.2) (layer "F.Cu") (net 3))
 (segment (start 132.1224 74.393) (end 135.068799 74.393) (width 0.2) (layer "F.Cu") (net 3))
 (segment (start 135.068799 74.393) (end 136.512999 72.9488) (width 0.2) (layer "F.Cu") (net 3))
 (segment (start 129.6634 76.852) (end 132.1224 74.393) (width 0.2) (layer "F.Cu") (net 3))
 (segment (start 136.512999 72.9488) (end 136.7028 72.9488) (width 0.2) (layer "F.Cu") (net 3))
 (via (at 136.7028 72.9488) (size 0.6) (drill 0.3) (layers "F.Cu" "B.Cu") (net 3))
 (via (at 132.7912 86.0044) (size 0.6) (drill 0.3) (layers "F.Cu" "B.Cu") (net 3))
 (segment (start 137.085 72.326) (end 136.7028 72.9488) (width 0.2) (layer "B.Cu") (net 3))
 (segment (start 137.2108 73.4568) (end 136.7028 72.9488) (width 0.2) (layer "B.Cu") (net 3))
 (segment (start 137.185 70.62) (end 137.185 71.632501) (width 0.2) (layer "B.Cu") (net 3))
 (segment (start 146.284 76.454) (end 138.2268 76.454) (width 0.2) (layer "B.Cu") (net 3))
 (segment (start 132.7912 86.0044) (end 132.6896 86.1858) (width 0.2) (layer "B.Cu") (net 3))
 (segment (start 137.185 71.632501) (end 137.085 71.732501) (width 0.2) (layer "B.Cu") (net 3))
 (segment (start 136.525 84.6) (end 136.935 85.01) (width 0.2) (layer "B.Cu") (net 3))
 (segment (start 136.5588 86.1858) (end 132.7912 86.0044) (width 0.2) (layer "B.Cu") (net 3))
 (segment (start 148.59 78.76) (end 146.284 76.454) (width 0.2) (layer "B.Cu") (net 3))
 (segment (start 137.085 71.732501) (end 137.085 72.326) (width 0.2) (layer "B.Cu") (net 3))
 (segment (start 138.2268 76.454) (end 137.2108 75.438) (width 0.2) (layer "B.Cu") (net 3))
 (segment (start 136.935 85.01) (end 136.935 85.8096) (width 0.2) (layer "B.Cu") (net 3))
 (segment (start 137.2108 75.438) (end 137.2108 73.4568) (width 0.2) (layer "B.Cu") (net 3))
 (segment (start 136.935 85.8096) (end 136.5588 86.1858) (width 0.2) (layer "B.Cu") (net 3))
 (segment (start 136.525 83.9) (end 136.525 84.6) (width 0.2) (layer "B.Cu") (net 3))
 (segment (start 148.33 81.56) (end 148.59 81.3) (width 0.2) (layer "B.Cu") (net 4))
 (segment (start 145.415 81.56) (end 148.33 81.56) (width 0.2) (layer "B.Cu") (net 4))
 (segment (start 133.24 76.765) (end 133.985 77.51) (width 0.2) (layer "B.Cu") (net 1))
 (segment (start 133.985 77.51) (end 133.985 83.9) (width 0.2) (layer "B.Cu") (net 1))
 (segment (start 131.936 73.943) (end 134.882401 73.943) (width 0.2) (layer "F.Cu") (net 15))
 (segment (start 132.7912 86.8172) (end 132.609801 86.635801) (width 0.2) (layer "F.Cu") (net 15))
 (segment (start 134.882401 73.943) (end 136.1948 72.630601) (width 0.2) (layer "F.Cu") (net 15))
 (segment (start 131.631201 86.635801) (end 129.2134 84.218) (width 0.2) (layer "F.Cu") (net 15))
 (segment (start 136.1948 72.630601) (end 136.1948 72.2884) (width 0.2) (layer "F.Cu") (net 15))
 (segment (start 129.2134 84.218) (end 129.2134 76.6656) (width 0.2) (layer "F.Cu") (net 15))
 (segment (start 132.609801 86.635801) (end 131.631201 86.635801) (width 0.2) (layer "F.Cu") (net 15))
 (segment (start 129.2134 76.6656) (end 131.936 73.943) (width 0.2) (layer "F.Cu") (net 15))
 (via (at 132.7912 86.8172) (size 0.6) (drill 0.3) (layers "F.Cu" "B.Cu") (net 15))
 (via (at 136.1948 72.2884) (size 0.6) (drill 0.3) (layers "F.Cu" "B.Cu") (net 15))
 (segment (start 136.7452 86.6358) (end 132.7912 86.8172) (width 0.2) (layer "B.Cu") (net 15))
 (segment (start 136.535 71.632501) (end 136.635 71.732501) (width 0.2) (layer "B.Cu") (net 15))
 (segment (start 137.385 85.01) (end 137.385 85.996) (width 0.2) (layer "B.Cu") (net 15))
 (segment (start 136.635 71.732501) (end 136.635 72.1396) (width 0.2) (layer "B.Cu") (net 15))
 (segment (start 136.635 72.1396) (end 136.1948 72.2884) (width 0.2) (layer "B.Cu") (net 15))
 (segment (start 137.385 85.996) (end 136.7452 86.6358) (width 0.2) (layer "B.Cu") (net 15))
 (segment (start 136.535 70.62) (end 136.535 71.632501) (width 0.2) (layer "B.Cu") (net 15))
 (segment (start 132.7912 86.8172) (end 132.6896 86.6358) (width 0.2) (layer "B.Cu") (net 15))
 (segment (start 134.9756 73.5076) (end 136.1948 72.2884) (width 0.2) (layer "B.Cu") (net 15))
 (segment (start 137.795 83.9) (end 137.795 84.6) (width 0.2) (layer "B.Cu") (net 15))
 (segment (start 137.795 84.6) (end 137.385 85.01) (width 0.2) (layer "B.Cu") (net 15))
 (segment (start 134.9756 73.8632) (end 134.9756 73.5076) (width 0.2) (layer "B.Cu") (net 15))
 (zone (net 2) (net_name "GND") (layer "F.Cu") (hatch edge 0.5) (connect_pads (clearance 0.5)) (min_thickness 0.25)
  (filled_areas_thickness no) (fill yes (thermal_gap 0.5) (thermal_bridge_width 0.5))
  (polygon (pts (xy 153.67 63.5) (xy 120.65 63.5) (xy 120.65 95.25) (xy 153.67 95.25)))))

